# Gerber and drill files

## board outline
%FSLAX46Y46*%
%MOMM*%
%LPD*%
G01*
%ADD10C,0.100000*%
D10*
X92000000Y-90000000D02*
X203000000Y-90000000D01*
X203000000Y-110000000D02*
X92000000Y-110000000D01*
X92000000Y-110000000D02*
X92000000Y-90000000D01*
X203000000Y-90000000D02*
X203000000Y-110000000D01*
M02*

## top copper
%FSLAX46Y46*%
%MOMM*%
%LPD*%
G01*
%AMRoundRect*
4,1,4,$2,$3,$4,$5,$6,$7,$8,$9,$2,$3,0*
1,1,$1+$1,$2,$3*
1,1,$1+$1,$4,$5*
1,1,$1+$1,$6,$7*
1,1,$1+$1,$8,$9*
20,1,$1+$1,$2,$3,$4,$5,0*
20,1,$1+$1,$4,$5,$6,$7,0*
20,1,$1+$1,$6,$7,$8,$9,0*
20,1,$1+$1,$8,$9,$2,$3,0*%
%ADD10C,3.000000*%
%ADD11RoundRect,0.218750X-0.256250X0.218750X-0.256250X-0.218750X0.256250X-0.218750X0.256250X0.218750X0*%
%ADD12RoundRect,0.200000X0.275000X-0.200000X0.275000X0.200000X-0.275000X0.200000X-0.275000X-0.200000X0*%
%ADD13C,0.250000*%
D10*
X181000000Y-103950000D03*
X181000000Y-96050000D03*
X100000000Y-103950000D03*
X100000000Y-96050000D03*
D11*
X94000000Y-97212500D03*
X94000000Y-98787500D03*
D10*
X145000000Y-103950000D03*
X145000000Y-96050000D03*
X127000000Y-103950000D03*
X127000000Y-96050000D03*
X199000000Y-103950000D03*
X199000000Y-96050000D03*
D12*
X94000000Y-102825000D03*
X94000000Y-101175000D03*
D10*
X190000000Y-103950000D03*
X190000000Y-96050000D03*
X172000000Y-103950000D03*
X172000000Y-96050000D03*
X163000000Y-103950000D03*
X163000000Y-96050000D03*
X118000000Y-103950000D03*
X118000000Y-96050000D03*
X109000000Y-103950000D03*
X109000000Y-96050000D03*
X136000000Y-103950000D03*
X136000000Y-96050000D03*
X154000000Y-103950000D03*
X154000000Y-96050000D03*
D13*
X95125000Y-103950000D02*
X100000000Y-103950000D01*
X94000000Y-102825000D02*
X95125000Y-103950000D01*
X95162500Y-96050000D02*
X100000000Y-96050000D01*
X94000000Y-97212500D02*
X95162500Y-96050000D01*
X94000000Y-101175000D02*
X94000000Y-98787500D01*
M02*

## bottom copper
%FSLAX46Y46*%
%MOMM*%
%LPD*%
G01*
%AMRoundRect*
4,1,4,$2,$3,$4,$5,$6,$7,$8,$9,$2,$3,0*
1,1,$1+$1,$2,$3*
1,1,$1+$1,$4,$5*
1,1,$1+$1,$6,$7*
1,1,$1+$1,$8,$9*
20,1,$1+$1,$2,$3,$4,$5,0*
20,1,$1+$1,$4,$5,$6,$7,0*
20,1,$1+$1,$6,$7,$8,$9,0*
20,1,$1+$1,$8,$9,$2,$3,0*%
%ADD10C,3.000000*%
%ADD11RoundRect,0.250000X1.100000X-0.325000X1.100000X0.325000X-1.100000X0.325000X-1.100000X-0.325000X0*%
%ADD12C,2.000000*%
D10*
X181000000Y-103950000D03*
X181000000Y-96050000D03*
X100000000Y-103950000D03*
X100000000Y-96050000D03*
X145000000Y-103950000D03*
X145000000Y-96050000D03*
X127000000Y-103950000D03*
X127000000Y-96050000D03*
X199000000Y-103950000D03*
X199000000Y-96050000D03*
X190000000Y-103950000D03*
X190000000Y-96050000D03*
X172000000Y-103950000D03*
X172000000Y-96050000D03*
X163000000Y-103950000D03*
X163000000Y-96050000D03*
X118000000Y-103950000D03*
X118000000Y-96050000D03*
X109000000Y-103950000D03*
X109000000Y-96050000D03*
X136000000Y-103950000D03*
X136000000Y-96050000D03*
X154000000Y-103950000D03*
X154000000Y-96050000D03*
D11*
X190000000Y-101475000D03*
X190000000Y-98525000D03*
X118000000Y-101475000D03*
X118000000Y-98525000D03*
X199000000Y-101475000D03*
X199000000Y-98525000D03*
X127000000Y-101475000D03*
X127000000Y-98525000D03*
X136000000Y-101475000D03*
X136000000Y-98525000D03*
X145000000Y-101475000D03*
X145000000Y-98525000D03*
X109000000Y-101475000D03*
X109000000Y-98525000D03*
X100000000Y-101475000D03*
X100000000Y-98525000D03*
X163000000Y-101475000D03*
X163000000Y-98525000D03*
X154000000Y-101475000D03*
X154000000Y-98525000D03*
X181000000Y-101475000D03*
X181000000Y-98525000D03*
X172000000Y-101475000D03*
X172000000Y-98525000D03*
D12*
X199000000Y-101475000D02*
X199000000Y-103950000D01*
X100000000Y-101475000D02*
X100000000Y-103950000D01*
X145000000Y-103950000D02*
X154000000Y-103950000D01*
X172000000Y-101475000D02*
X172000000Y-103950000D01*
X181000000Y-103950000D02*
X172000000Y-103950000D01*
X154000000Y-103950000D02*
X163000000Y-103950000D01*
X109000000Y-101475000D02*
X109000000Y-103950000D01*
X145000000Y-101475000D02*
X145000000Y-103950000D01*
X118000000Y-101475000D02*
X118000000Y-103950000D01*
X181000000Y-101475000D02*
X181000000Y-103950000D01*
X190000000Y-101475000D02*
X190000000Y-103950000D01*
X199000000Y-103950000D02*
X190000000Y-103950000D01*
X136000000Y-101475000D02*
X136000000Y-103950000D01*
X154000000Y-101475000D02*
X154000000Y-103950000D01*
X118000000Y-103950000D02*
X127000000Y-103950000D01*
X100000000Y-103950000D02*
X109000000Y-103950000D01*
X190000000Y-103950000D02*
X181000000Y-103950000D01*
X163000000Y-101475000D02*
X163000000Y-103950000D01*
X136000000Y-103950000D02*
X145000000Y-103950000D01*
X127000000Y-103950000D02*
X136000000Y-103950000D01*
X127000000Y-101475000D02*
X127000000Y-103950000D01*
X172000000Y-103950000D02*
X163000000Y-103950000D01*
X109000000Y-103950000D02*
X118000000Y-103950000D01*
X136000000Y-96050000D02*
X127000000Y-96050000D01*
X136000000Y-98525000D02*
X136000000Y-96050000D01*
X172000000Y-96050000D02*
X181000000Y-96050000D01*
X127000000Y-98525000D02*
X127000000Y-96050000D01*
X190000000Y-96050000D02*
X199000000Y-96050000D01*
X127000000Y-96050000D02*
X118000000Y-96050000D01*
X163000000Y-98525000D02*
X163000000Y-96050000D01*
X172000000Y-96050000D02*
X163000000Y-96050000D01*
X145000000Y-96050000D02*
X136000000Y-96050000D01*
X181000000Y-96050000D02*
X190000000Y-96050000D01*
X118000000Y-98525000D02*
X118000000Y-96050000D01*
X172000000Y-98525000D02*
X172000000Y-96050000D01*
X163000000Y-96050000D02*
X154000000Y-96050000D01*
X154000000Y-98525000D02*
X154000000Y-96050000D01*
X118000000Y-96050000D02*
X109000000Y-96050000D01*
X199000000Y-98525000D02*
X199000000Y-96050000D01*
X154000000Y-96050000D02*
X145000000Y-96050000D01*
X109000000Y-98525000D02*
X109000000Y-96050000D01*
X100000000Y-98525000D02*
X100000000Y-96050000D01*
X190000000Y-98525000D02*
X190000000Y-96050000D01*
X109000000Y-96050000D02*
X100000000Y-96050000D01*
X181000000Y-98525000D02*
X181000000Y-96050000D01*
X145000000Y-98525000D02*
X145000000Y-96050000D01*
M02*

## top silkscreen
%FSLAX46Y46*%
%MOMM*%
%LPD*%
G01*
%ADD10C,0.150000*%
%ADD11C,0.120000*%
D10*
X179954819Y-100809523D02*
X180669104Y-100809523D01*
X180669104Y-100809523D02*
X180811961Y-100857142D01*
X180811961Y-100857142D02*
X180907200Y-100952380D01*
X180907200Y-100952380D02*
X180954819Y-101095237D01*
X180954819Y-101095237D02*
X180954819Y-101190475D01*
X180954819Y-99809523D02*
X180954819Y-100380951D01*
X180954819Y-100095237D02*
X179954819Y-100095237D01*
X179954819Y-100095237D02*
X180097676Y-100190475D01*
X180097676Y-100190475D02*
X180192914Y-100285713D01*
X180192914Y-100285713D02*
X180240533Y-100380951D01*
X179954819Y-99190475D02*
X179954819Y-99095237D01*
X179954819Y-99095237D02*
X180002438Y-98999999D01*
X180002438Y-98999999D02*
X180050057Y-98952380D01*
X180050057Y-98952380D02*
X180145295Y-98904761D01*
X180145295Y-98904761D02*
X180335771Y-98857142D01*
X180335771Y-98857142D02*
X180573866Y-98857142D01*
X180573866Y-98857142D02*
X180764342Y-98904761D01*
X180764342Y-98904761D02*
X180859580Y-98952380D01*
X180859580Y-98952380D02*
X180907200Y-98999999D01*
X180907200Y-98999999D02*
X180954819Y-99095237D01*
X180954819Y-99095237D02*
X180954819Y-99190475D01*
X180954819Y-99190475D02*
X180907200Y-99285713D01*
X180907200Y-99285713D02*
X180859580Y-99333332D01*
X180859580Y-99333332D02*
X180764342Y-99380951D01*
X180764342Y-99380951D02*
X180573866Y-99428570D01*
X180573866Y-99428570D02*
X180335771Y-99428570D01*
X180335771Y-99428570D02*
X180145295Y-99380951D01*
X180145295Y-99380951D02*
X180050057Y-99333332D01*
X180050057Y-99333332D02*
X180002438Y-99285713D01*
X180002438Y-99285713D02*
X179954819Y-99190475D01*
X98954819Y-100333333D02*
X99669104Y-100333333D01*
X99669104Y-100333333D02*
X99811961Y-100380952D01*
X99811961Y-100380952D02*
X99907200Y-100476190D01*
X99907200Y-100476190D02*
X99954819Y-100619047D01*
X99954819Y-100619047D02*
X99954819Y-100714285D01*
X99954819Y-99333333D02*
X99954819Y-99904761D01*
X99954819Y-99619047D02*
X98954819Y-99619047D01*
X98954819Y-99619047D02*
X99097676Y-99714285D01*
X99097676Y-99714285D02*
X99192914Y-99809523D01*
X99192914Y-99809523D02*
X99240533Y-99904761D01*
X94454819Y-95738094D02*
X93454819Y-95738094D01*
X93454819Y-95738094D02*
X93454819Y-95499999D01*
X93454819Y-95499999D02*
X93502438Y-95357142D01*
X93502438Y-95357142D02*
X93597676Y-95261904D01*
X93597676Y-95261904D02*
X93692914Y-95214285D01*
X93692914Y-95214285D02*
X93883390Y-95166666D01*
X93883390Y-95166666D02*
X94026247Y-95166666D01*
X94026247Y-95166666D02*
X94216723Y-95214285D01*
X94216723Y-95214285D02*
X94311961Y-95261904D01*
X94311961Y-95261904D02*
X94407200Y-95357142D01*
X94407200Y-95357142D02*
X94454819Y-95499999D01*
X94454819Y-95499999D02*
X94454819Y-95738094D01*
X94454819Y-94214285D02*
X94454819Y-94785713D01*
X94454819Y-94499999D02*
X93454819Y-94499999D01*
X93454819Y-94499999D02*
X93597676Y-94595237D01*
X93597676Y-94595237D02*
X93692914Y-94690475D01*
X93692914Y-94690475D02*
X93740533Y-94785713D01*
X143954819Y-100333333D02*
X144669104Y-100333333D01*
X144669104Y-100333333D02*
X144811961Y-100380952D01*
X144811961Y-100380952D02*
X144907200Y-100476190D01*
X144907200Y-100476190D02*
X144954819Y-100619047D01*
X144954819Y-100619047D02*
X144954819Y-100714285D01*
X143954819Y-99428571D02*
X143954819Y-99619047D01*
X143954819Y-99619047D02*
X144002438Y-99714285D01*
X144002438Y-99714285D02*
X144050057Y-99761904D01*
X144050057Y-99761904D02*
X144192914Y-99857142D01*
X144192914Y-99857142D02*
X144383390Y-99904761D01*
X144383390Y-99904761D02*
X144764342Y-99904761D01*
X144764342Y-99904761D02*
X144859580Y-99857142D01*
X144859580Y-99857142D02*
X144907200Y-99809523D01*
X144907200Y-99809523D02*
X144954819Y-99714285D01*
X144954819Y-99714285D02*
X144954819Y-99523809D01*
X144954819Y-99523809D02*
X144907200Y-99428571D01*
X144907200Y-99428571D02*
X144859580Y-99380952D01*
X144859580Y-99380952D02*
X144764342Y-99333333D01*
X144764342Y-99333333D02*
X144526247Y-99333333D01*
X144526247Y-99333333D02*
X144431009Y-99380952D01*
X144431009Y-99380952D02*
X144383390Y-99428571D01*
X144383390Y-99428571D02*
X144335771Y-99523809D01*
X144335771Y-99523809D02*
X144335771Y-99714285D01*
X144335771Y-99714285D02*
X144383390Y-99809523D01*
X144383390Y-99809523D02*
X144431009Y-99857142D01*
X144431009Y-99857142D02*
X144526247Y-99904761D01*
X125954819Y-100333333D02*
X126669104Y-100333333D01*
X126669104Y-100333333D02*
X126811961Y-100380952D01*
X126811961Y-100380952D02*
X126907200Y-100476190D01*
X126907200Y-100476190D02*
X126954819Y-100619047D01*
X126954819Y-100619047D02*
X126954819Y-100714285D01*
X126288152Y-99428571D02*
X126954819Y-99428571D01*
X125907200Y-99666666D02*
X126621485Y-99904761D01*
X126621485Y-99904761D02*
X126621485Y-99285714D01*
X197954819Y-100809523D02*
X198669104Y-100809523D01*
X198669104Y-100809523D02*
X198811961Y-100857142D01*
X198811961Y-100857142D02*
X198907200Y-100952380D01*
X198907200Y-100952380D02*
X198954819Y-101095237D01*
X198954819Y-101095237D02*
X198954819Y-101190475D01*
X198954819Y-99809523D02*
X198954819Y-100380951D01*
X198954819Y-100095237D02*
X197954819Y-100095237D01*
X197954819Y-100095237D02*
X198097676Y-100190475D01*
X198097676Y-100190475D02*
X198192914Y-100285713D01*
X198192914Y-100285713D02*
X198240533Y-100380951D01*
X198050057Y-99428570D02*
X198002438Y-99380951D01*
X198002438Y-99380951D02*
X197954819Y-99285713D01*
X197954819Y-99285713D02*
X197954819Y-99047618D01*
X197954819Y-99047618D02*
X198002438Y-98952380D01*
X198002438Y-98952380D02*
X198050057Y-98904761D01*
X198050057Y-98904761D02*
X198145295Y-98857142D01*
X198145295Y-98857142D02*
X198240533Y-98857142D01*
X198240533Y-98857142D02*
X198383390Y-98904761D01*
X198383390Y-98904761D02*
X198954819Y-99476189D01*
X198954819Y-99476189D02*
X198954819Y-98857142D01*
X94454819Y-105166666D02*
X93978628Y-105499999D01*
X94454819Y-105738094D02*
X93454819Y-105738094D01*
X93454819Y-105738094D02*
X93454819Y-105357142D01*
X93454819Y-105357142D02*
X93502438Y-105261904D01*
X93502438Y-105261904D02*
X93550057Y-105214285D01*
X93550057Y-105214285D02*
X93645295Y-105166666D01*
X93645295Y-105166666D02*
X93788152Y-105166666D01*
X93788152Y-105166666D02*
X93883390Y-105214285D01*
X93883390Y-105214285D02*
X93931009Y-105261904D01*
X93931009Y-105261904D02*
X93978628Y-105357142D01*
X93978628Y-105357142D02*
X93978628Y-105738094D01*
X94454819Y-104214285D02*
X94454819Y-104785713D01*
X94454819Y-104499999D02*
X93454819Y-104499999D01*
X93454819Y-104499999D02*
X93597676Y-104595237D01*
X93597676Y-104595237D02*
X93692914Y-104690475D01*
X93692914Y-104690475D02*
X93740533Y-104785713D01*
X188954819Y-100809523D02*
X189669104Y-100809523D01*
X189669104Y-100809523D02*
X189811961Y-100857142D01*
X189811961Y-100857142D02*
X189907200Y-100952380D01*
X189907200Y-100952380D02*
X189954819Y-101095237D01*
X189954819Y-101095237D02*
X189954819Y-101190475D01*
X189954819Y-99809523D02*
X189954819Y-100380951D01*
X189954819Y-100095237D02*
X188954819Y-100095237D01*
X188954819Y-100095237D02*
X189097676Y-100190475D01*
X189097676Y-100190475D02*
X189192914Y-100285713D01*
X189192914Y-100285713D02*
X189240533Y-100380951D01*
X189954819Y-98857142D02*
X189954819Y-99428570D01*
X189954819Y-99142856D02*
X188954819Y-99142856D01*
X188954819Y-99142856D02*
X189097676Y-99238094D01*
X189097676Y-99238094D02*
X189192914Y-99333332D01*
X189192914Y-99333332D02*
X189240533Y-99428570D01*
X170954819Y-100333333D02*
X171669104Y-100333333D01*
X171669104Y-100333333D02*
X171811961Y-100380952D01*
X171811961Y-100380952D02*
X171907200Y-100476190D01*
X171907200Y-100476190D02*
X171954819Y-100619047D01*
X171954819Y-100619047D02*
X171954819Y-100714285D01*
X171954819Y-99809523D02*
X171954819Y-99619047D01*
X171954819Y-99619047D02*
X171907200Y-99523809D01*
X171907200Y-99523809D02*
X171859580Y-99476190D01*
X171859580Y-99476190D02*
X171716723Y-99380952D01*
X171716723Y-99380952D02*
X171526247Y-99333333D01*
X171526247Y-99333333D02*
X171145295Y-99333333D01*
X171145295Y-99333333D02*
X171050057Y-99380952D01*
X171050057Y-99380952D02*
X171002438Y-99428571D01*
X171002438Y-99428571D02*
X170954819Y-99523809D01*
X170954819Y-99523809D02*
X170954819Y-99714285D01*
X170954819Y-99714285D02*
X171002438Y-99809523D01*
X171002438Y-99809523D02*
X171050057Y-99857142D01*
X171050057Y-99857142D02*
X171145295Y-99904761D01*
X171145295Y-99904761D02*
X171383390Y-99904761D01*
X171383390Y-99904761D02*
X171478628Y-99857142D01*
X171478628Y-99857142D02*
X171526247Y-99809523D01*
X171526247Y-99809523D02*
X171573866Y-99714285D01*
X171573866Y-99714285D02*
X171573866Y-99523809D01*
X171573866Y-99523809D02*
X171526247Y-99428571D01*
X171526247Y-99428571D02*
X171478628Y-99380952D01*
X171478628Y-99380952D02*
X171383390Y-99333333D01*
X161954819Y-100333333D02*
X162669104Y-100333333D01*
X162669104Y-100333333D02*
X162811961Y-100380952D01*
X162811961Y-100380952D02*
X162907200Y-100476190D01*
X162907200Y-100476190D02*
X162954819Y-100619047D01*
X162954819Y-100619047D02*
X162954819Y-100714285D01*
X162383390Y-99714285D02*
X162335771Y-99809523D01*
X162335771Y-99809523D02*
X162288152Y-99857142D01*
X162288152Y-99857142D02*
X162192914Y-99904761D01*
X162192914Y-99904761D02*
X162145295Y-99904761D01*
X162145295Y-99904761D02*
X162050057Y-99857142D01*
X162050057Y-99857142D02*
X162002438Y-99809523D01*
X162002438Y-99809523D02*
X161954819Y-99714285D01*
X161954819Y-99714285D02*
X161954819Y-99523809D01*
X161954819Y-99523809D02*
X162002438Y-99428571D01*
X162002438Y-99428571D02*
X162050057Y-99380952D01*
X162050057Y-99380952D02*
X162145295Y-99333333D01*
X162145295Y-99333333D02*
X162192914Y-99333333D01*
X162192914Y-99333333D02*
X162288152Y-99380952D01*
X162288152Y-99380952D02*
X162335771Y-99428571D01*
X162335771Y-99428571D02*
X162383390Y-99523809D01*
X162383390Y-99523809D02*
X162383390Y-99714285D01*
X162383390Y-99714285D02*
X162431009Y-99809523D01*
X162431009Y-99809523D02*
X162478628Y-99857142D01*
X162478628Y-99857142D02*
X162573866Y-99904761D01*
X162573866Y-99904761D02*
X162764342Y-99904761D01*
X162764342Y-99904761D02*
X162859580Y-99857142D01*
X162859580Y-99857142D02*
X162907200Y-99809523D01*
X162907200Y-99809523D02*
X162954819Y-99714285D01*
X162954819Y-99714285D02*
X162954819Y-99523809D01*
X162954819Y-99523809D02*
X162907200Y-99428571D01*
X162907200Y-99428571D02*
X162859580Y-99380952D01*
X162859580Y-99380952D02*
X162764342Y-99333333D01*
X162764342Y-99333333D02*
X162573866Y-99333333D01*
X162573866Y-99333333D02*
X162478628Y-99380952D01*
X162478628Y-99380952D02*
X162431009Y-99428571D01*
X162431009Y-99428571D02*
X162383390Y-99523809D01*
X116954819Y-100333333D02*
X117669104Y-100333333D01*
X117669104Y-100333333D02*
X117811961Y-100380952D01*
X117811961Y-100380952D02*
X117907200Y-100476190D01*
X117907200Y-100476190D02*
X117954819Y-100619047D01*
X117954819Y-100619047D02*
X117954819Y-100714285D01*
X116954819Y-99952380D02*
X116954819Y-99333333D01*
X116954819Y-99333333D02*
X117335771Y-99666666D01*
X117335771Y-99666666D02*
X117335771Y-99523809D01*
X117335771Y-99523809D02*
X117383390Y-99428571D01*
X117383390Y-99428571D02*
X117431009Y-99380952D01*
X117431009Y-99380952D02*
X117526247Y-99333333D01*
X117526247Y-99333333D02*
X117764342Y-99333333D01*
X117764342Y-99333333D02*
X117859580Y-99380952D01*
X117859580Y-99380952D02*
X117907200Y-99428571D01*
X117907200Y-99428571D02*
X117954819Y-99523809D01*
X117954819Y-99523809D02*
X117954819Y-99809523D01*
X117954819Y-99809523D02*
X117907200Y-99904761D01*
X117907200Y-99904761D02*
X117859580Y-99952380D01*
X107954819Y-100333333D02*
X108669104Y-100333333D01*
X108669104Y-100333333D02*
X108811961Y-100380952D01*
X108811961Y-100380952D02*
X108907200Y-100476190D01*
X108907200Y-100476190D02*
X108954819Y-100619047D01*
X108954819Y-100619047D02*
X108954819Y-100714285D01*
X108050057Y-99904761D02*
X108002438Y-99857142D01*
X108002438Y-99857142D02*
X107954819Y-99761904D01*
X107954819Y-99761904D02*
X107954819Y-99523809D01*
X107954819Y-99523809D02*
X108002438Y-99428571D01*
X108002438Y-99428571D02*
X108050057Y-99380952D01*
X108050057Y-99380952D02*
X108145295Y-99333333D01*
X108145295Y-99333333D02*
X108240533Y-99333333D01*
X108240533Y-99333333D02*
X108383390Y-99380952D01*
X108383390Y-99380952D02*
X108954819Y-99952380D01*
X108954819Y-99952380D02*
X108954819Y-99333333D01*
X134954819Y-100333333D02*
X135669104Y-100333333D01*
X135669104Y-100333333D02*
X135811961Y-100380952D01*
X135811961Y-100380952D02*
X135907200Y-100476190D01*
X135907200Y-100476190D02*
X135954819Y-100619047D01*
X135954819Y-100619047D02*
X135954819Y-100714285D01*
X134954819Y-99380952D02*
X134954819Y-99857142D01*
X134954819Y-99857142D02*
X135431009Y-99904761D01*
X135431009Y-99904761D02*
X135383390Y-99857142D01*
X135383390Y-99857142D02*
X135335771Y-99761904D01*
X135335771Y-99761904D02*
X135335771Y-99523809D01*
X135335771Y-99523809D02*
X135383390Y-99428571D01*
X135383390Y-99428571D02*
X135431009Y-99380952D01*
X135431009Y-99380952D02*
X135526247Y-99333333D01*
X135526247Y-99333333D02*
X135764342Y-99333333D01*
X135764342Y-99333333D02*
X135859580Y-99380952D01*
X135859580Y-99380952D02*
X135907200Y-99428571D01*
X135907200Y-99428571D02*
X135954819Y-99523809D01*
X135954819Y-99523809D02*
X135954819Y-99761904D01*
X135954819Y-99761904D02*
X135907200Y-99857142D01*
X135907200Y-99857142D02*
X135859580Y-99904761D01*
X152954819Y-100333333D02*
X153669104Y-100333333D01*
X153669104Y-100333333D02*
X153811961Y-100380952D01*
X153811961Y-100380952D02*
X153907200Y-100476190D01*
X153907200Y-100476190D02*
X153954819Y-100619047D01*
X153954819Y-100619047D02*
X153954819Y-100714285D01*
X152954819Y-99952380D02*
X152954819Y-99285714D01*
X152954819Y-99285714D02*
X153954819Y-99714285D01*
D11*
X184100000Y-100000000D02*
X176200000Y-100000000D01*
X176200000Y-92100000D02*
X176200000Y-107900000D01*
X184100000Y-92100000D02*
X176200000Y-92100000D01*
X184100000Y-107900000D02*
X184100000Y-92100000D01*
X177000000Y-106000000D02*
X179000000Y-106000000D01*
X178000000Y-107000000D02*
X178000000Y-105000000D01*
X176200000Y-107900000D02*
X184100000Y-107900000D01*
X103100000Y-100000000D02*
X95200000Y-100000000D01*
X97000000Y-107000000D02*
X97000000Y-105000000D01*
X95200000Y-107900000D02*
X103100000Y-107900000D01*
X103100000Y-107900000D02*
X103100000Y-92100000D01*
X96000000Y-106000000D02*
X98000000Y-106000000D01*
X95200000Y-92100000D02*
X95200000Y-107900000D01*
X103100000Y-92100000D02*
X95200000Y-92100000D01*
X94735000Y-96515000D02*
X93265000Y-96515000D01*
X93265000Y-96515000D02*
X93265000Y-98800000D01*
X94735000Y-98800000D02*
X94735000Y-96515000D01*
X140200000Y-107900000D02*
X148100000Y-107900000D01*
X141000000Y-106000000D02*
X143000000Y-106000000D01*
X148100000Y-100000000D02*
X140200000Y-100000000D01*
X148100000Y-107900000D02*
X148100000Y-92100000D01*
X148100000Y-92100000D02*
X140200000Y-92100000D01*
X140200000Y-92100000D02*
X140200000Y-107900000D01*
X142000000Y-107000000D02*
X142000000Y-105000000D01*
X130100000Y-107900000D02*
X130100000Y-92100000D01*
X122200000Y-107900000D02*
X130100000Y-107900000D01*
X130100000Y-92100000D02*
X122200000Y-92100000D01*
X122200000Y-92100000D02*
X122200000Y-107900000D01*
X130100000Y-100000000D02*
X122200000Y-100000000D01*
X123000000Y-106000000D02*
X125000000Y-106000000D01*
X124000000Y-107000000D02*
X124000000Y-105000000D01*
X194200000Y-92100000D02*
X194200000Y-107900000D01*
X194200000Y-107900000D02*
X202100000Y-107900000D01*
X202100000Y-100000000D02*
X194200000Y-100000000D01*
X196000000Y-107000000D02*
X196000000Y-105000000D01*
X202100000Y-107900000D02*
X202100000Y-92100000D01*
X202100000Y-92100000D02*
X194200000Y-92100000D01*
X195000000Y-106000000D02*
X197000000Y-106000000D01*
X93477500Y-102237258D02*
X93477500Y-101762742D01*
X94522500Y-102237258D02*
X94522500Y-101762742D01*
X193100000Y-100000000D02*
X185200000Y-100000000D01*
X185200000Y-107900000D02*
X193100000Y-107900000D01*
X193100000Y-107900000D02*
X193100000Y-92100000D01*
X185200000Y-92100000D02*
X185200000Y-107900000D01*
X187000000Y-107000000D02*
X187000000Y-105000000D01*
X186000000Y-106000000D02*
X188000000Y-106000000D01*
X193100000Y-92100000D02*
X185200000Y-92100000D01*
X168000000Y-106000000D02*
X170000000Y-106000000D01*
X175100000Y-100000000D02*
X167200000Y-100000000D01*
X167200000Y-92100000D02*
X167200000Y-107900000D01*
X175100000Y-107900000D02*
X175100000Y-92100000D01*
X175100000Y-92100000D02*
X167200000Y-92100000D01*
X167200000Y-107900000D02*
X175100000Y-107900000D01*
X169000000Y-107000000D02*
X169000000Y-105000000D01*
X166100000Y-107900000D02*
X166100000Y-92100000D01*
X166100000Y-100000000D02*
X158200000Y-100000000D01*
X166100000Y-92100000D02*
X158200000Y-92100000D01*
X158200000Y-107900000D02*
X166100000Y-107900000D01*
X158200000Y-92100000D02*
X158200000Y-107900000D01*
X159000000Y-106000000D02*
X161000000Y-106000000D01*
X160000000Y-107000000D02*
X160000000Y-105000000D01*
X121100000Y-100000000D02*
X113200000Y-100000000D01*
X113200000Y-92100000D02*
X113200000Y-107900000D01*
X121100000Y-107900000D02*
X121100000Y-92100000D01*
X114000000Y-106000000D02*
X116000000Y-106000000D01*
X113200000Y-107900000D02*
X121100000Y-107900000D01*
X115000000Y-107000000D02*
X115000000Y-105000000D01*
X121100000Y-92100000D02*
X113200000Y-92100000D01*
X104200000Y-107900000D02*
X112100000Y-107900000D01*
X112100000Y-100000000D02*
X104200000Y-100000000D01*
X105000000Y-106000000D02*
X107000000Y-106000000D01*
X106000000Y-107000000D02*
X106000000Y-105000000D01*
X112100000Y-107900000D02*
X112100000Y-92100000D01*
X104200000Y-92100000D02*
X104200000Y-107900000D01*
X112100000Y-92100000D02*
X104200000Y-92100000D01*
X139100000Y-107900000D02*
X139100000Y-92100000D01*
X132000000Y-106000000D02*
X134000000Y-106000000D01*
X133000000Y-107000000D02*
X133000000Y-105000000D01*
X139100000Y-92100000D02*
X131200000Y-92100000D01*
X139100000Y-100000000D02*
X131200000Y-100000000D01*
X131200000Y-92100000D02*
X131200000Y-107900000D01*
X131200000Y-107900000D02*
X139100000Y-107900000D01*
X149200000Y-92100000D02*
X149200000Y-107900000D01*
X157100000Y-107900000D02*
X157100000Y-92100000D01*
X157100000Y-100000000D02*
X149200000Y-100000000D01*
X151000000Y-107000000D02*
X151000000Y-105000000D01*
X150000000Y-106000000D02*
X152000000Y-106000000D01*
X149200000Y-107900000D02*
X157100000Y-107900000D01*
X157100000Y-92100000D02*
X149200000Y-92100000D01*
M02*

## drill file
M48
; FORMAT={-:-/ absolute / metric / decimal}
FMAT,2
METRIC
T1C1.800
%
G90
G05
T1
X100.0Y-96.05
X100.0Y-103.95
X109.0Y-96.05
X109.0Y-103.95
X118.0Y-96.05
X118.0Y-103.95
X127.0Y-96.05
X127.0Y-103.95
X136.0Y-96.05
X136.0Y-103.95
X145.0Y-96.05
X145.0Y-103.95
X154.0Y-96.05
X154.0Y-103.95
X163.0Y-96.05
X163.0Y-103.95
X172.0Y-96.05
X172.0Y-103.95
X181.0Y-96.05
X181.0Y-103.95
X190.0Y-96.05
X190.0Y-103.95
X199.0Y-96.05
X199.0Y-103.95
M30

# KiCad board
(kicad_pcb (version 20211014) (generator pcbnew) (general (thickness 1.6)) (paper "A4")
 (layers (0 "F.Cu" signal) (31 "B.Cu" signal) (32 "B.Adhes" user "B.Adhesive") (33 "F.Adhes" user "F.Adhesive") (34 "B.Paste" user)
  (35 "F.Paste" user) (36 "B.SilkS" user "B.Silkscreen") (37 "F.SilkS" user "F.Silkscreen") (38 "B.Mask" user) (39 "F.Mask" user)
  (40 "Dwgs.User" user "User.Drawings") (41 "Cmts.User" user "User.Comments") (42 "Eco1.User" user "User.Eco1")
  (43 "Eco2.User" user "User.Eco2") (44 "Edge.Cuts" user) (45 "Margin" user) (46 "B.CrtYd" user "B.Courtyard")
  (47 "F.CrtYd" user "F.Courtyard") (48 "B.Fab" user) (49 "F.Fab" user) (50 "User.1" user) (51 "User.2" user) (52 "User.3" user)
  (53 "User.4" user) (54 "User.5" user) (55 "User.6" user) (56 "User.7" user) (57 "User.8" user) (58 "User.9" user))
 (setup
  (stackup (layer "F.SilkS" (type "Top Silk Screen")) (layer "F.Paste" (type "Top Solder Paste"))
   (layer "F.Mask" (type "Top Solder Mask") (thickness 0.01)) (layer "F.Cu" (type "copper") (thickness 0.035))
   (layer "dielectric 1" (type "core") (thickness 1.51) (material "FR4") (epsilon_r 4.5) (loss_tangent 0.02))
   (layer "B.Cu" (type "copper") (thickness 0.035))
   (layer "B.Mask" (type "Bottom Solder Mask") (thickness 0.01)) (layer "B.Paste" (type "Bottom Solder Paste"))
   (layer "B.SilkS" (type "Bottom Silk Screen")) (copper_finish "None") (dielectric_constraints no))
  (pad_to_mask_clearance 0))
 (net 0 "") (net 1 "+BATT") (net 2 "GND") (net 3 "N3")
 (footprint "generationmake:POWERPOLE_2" (layer "F.Cu") (at 181 100 90)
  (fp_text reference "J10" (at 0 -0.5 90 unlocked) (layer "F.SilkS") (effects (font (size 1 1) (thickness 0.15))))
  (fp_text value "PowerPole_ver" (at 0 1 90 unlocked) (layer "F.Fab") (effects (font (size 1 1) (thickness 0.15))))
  (fp_line (start 0 3.1) (end 0 -4.8) (layer "F.SilkS") (width 0.12))
  (fp_line (start 7.9 -4.8) (end -7.9 -4.8) (layer "F.SilkS") (width 0.12))
  (fp_line (start 7.9 3.1) (end 7.9 -4.8) (layer "F.SilkS") (width 0.12))
  (fp_line (start -7.9 3.1) (end 7.9 3.1) (layer "F.SilkS") (width 0.12))
  (fp_line (start -6 -4) (end -6 -2) (layer "F.SilkS") (width 0.12))
  (fp_line (start -7 -3) (end -5 -3) (layer "F.SilkS") (width 0.12))
  (fp_line (start -7.9 -4.8) (end -7.9 3.1) (layer "F.SilkS") (width 0.12))
  (pad "1" thru_hole circle (at -3.95 0 90) (size 3 3) (drill 1.8) (layers *.Cu *.Mask) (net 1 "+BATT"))
  (pad "2" thru_hole circle (at 3.95 0 90) (size 3 3) (drill 1.8) (layers *.Cu *.Mask) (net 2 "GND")))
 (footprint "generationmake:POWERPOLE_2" (layer "F.Cu") (at 100 100 90)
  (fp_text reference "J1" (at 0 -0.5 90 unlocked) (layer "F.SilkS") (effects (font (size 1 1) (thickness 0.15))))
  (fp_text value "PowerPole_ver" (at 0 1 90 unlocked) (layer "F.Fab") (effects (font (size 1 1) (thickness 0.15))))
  (fp_line (start 0 3.1) (end 0 -4.8) (layer "F.SilkS") (width 0.12))
  (fp_line (start -7 -3) (end -5 -3) (layer "F.SilkS") (width 0.12))
  (fp_line (start -7.9 -4.8) (end -7.9 3.1) (layer "F.SilkS") (width 0.12))
  (fp_line (start -7.9 3.1) (end 7.9 3.1) (layer "F.SilkS") (width 0.12))
  (fp_line (start -6 -4) (end -6 -2) (layer "F.SilkS") (width 0.12))
  (fp_line (start 7.9 -4.8) (end -7.9 -4.8) (layer "F.SilkS") (width 0.12))
  (fp_line (start 7.9 3.1) (end 7.9 -4.8) (layer "F.SilkS") (width 0.12))
  (pad "1" thru_hole circle (at -3.95 0 90) (size 3 3) (drill 1.8) (layers *.Cu *.Mask) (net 1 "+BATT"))
  (pad "2" thru_hole circle (at 3.95 0 90) (size 3 3) (drill 1.8) (layers *.Cu *.Mask) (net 2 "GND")))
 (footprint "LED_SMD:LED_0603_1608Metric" (layer "F.Cu") (at 94 98 -90)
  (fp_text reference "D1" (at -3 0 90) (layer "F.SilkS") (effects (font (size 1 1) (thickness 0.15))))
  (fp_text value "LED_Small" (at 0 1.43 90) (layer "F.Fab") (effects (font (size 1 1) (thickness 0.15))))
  (fp_line (start -1.485 -0.735) (end -1.485 0.735) (layer "F.SilkS") (width 0.12))
  (fp_line (start -1.485 0.735) (end 0.8 0.735) (layer "F.SilkS") (width 0.12))
  (fp_line (start 0.8 -0.735) (end -1.485 -0.735) (layer "F.SilkS") (width 0.12))
  (pad "1" smd roundrect (at -0.7875 0 270) (size 0.875 0.95) (layers "F.Cu" "F.Paste" "F.Mask") (roundrect_rratio 0.25) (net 2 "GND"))
  (pad "2" smd roundrect (at 0.7875 0 270) (size 0.875 0.95) (layers "F.Cu" "F.Paste" "F.Mask") (roundrect_rratio 0.25) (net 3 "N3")))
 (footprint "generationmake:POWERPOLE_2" (layer "F.Cu") (at 145 100 90)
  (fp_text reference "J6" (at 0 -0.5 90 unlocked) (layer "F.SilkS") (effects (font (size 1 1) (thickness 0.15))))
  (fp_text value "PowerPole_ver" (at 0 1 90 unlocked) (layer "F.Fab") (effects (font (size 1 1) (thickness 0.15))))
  (fp_line (start -7.9 -4.8) (end -7.9 3.1) (layer "F.SilkS") (width 0.12))
  (fp_line (start -6 -4) (end -6 -2) (layer "F.SilkS") (width 0.12))
  (fp_line (start 0 3.1) (end 0 -4.8) (layer "F.SilkS") (width 0.12))
  (fp_line (start -7.9 3.1) (end 7.9 3.1) (layer "F.SilkS") (width 0.12))
  (fp_line (start 7.9 3.1) (end 7.9 -4.8) (layer "F.SilkS") (width 0.12))
  (fp_line (start 7.9 -4.8) (end -7.9 -4.8) (layer "F.SilkS") (width 0.12))
  (fp_line (start -7 -3) (end -5 -3) (layer "F.SilkS") (width 0.12))
  (pad "1" thru_hole circle (at -3.95 0 90) (size 3 3) (drill 1.8) (layers *.Cu *.Mask) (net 1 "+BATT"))
  (pad "2" thru_hole circle (at 3.95 0 90) (size 3 3) (drill 1.8) (layers *.Cu *.Mask) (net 2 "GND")))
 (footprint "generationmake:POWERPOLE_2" (layer "F.Cu") (at 127 100 90)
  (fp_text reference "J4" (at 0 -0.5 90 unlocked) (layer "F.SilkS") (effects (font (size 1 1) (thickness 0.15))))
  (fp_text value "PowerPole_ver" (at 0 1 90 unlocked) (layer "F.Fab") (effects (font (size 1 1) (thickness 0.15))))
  (fp_line (start -7.9 3.1) (end 7.9 3.1) (layer "F.SilkS") (width 0.12))
  (fp_line (start -7.9 -4.8) (end -7.9 3.1) (layer "F.SilkS") (width 0.12))
  (fp_line (start 7.9 3.1) (end 7.9 -4.8) (layer "F.SilkS") (width 0.12))
  (fp_line (start 7.9 -4.8) (end -7.9 -4.8) (layer "F.SilkS") (width 0.12))
  (fp_line (start 0 3.1) (end 0 -4.8) (layer "F.SilkS") (width 0.12))
  (fp_line (start -6 -4) (end -6 -2) (layer "F.SilkS") (width 0.12))
  (fp_line (start -7 -3) (end -5 -3) (layer "F.SilkS") (width 0.12))
  (pad "1" thru_hole circle (at -3.95 0 90) (size 3 3) (drill 1.8) (layers *.Cu *.Mask) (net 1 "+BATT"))
  (pad "2" thru_hole circle (at 3.95 0 90) (size 3 3) (drill 1.8) (layers *.Cu *.Mask) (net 2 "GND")))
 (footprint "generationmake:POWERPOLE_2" (layer "F.Cu") (at 199 100 90)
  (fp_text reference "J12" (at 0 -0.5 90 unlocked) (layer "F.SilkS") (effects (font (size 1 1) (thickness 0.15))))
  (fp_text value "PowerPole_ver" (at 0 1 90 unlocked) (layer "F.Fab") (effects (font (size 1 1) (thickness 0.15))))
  (fp_line (start 7.9 -4.8) (end -7.9 -4.8) (layer "F.SilkS") (width 0.12))
  (fp_line (start -7.9 -4.8) (end -7.9 3.1) (layer "F.SilkS") (width 0.12))
  (fp_line (start 0 3.1) (end 0 -4.8) (layer "F.SilkS") (width 0.12))
  (fp_line (start -7 -3) (end -5 -3) (layer "F.SilkS") (width 0.12))
  (fp_line (start -7.9 3.1) (end 7.9 3.1) (layer "F.SilkS") (width 0.12))
  (fp_line (start 7.9 3.1) (end 7.9 -4.8) (layer "F.SilkS") (width 0.12))
  (fp_line (start -6 -4) (end -6 -2) (layer "F.SilkS") (width 0.12))
  (pad "1" thru_hole circle (at -3.95 0 90) (size 3 3) (drill 1.8) (layers *.Cu *.Mask) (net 1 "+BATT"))
  (pad "2" thru_hole circle (at 3.95 0 90) (size 3 3) (drill 1.8) (layers *.Cu *.Mask) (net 2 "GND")))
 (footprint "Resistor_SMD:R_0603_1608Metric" (layer "F.Cu") (at 94 102 90)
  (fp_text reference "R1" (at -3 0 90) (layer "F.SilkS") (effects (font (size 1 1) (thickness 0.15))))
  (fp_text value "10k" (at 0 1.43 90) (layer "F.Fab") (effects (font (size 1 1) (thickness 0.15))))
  (fp_line (start -0.237258 -0.5225) (end 0.237258 -0.5225) (layer "F.SilkS") (width 0.12))
  (fp_line (start -0.237258 0.5225) (end 0.237258 0.5225) (layer "F.SilkS") (width 0.12))
  (pad "1" smd roundrect (at -0.825 0 90) (size 0.8 0.95) (layers "F.Cu" "F.Paste" "F.Mask") (roundrect_rratio 0.25) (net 1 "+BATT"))
  (pad "2" smd roundrect (at 0.825 0 90) (size 0.8 0.95) (layers "F.Cu" "F.Paste" "F.Mask") (roundrect_rratio 0.25) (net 3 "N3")))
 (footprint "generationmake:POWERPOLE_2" (layer "F.Cu") (at 190 100 90)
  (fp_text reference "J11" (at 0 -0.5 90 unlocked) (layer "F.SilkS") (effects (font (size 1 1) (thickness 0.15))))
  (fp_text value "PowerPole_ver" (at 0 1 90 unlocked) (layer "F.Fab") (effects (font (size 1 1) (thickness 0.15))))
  (fp_line (start 0 3.1) (end 0 -4.8) (layer "F.SilkS") (width 0.12))
  (fp_line (start -7.9 -4.8) (end -7.9 3.1) (layer "F.SilkS") (width 0.12))
  (fp_line (start -7.9 3.1) (end 7.9 3.1) (layer "F.SilkS") (width 0.12))
  (fp_line (start 7.9 -4.8) (end -7.9 -4.8) (layer "F.SilkS") (width 0.12))
  (fp_line (start -7 -3) (end -5 -3) (layer "F.SilkS") (width 0.12))
  (fp_line (start -6 -4) (end -6 -2) (layer "F.SilkS") (width 0.12))
  (fp_line (start 7.9 3.1) (end 7.9 -4.8) (layer "F.SilkS") (width 0.12))
  (pad "1" thru_hole circle (at -3.95 0 90) (size 3 3) (drill 1.8) (layers *.Cu *.Mask) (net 1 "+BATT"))
  (pad "2" thru_hole circle (at 3.95 0 90) (size 3 3) (drill 1.8) (layers *.Cu *.Mask) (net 2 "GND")))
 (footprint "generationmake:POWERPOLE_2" (layer "F.Cu") (at 172 100 90)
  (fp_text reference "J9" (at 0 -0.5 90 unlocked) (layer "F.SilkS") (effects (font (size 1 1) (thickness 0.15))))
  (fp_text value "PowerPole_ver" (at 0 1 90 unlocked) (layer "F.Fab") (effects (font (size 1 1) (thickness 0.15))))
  (fp_line (start -6 -4) (end -6 -2) (layer "F.SilkS") (width 0.12))
  (fp_line (start 0 3.1) (end 0 -4.8) (layer "F.SilkS") (width 0.12))
  (fp_line (start 7.9 -4.8) (end -7.9 -4.8) (layer "F.SilkS") (width 0.12))
  (fp_line (start -7.9 3.1) (end 7.9 3.1) (layer "F.SilkS") (width 0.12))
  (fp_line (start 7.9 3.1) (end 7.9 -4.8) (layer "F.SilkS") (width 0.12))
  (fp_line (start -7.9 -4.8) (end -7.9 3.1) (layer "F.SilkS") (width 0.12))
  (fp_line (start -7 -3) (end -5 -3) (layer "F.SilkS") (width 0.12))
  (pad "1" thru_hole circle (at -3.95 0 90) (size 3 3) (drill 1.8) (layers *.Cu *.Mask) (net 1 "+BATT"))
  (pad "2" thru_hole circle (at 3.95 0 90) (size 3 3) (drill 1.8) (layers *.Cu *.Mask) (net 2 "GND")))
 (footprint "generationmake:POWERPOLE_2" (layer "F.Cu") (at 163 100 90)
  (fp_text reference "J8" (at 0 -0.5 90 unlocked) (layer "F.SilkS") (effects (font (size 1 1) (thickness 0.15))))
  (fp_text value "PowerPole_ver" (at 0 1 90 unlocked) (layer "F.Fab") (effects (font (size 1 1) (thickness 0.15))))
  (fp_line (start -7.9 3.1) (end 7.9 3.1) (layer "F.SilkS") (width 0.12))
  (fp_line (start 0 3.1) (end 0 -4.8) (layer "F.SilkS") (width 0.12))
  (fp_line (start 7.9 3.1) (end 7.9 -4.8) (layer "F.SilkS") (width 0.12))
  (fp_line (start -7.9 -4.8) (end -7.9 3.1) (layer "F.SilkS") (width 0.12))
  (fp_line (start 7.9 -4.8) (end -7.9 -4.8) (layer "F.SilkS") (width 0.12))
  (fp_line (start -6 -4) (end -6 -2) (layer "F.SilkS") (width 0.12))
  (fp_line (start -7 -3) (end -5 -3) (layer "F.SilkS") (width 0.12))
  (pad "1" thru_hole circle (at -3.95 0 90) (size 3 3) (drill 1.8) (layers *.Cu *.Mask) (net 1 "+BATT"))
  (pad "2" thru_hole circle (at 3.95 0 90) (size 3 3) (drill 1.8) (layers *.Cu *.Mask) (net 2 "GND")))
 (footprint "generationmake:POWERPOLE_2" (layer "F.Cu") (at 118 100 90)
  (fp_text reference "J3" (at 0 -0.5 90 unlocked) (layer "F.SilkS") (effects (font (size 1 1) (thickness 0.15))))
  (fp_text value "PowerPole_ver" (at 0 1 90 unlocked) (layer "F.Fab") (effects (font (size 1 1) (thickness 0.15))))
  (fp_line (start 0 3.1) (end 0 -4.8) (layer "F.SilkS") (width 0.12))
  (fp_line (start 7.9 -4.8) (end -7.9 -4.8) (layer "F.SilkS") (width 0.12))
  (fp_line (start -7.9 3.1) (end 7.9 3.1) (layer "F.SilkS") (width 0.12))
  (fp_line (start -6 -4) (end -6 -2) (layer "F.SilkS") (width 0.12))
  (fp_line (start -7.9 -4.8) (end -7.9 3.1) (layer "F.SilkS") (width 0.12))
  (fp_line (start -7 -3) (end -5 -3) (layer "F.SilkS") (width 0.12))
  (fp_line (start 7.9 3.1) (end 7.9 -4.8) (layer "F.SilkS") (width 0.12))
  (pad "1" thru_hole circle (at -3.95 0 90) (size 3 3) (drill 1.8) (layers *.Cu *.Mask) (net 1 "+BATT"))
  (pad "2" thru_hole circle (at 3.95 0 90) (size 3 3) (drill 1.8) (layers *.Cu *.Mask) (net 2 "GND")))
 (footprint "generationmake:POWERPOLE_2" (layer "F.Cu") (at 109 100 90)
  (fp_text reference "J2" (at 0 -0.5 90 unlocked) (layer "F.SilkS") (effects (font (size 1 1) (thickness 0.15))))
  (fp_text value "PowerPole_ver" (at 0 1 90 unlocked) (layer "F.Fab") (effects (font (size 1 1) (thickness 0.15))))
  (fp_line (start -7.9 -4.8) (end -7.9 3.1) (layer "F.SilkS") (width 0.12))
  (fp_line (start 0 3.1) (end 0 -4.8) (layer "F.SilkS") (width 0.12))
  (fp_line (start -6 -4) (end -6 -2) (layer "F.SilkS") (width 0.12))
  (fp_line (start -7 -3) (end -5 -3) (layer "F.SilkS") (width 0.12))
  (fp_line (start -7.9 3.1) (end 7.9 3.1) (layer "F.SilkS") (width 0.12))
  (fp_line (start 7.9 -4.8) (end -7.9 -4.8) (layer "F.SilkS") (width 0.12))
  (fp_line (start 7.9 3.1) (end 7.9 -4.8) (layer "F.SilkS") (width 0.12))
  (pad "1" thru_hole circle (at -3.95 0 90) (size 3 3) (drill 1.8) (layers *.Cu *.Mask) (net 1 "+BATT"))
  (pad "2" thru_hole circle (at 3.95 0 90) (size 3 3) (drill 1.8) (layers *.Cu *.Mask) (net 2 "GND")))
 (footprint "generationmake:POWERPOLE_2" (layer "F.Cu") (at 136 100 90)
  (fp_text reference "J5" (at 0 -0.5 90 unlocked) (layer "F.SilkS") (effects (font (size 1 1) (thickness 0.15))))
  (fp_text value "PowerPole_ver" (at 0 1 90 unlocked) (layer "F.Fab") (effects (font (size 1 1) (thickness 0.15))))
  (fp_line (start -7.9 3.1) (end 7.9 3.1) (layer "F.SilkS") (width 0.12))
  (fp_line (start -6 -4) (end -6 -2) (layer "F.SilkS") (width 0.12))
  (fp_line (start -7 -3) (end -5 -3) (layer "F.SilkS") (width 0.12))
  (fp_line (start 7.9 3.1) (end 7.9 -4.8) (layer "F.SilkS") (width 0.12))
  (fp_line (start 0 3.1) (end 0 -4.8) (layer "F.SilkS") (width 0.12))
  (fp_line (start 7.9 -4.8) (end -7.9 -4.8) (layer "F.SilkS") (width 0.12))
  (fp_line (start -7.9 -4.8) (end -7.9 3.1) (layer "F.SilkS") (width 0.12))
  (pad "1" thru_hole circle (at -3.95 0 90) (size 3 3) (drill 1.8) (layers *.Cu *.Mask) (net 1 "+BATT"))
  (pad "2" thru_hole circle (at 3.95 0 90) (size 3 3) (drill 1.8) (layers *.Cu *.Mask) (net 2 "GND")))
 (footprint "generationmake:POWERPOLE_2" (layer "F.Cu") (at 154 100 90)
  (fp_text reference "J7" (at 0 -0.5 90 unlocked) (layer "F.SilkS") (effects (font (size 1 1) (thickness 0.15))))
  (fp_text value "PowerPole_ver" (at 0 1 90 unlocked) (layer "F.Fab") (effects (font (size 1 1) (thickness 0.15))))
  (fp_line (start 7.9 -4.8) (end -7.9 -4.8) (layer "F.SilkS") (width 0.12))
  (fp_line (start -7.9 3.1) (end 7.9 3.1) (layer "F.SilkS") (width 0.12))
  (fp_line (start 0 3.1) (end 0 -4.8) (layer "F.SilkS") (width 0.12))
  (fp_line (start -7 -3) (end -5 -3) (layer "F.SilkS") (width 0.12))
  (fp_line (start -6 -4) (end -6 -2) (layer "F.SilkS") (width 0.12))
  (fp_line (start -7.9 -4.8) (end -7.9 3.1) (layer "F.SilkS") (width 0.12))
  (fp_line (start 7.9 3.1) (end 7.9 -4.8) (layer "F.SilkS") (width 0.12))
  (pad "1" thru_hole circle (at -3.95 0 90) (size 3 3) (drill 1.8) (layers *.Cu *.Mask) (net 1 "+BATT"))
  (pad "2" thru_hole circle (at 3.95 0 90) (size 3 3) (drill 1.8) (layers *.Cu *.Mask) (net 2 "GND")))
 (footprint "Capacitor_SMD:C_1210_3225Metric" (layer "B.Cu") (at 190 100 90)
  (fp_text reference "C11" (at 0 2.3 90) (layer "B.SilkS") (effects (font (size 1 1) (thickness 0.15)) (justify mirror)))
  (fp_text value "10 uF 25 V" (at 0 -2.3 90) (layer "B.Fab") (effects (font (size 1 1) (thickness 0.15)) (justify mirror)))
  (pad "1" smd roundrect (at -1.475 0 90) (size 1.15 2.7) (layers "B.Cu" "B.Paste" "B.Mask") (roundrect_rratio 0.217391) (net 1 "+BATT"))
  (pad "2" smd roundrect (at 1.475 0 90) (size 1.15 2.7) (layers "B.Cu" "B.Paste" "B.Mask") (roundrect_rratio 0.217391) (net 2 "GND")))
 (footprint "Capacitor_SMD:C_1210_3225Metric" (layer "B.Cu") (at 118 100 90)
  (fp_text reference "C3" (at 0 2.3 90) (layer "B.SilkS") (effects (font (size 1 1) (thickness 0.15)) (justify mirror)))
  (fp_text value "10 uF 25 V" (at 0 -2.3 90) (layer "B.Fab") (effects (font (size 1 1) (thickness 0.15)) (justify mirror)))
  (pad "1" smd roundrect (at -1.475 0 90) (size 1.15 2.7) (layers "B.Cu" "B.Paste" "B.Mask") (roundrect_rratio 0.217391) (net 1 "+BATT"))
  (pad "2" smd roundrect (at 1.475 0 90) (size 1.15 2.7) (layers "B.Cu" "B.Paste" "B.Mask") (roundrect_rratio 0.217391) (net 2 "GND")))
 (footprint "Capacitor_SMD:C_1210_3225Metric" (layer "B.Cu") (at 199 100 90)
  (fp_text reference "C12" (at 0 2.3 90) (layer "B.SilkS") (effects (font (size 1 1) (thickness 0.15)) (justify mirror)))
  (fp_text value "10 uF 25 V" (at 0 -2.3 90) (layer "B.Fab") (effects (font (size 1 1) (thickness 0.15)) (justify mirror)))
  (pad "1" smd roundrect (at -1.475 0 90) (size 1.15 2.7) (layers "B.Cu" "B.Paste" "B.Mask") (roundrect_rratio 0.217391) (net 1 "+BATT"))
  (pad "2" smd roundrect (at 1.475 0 90) (size 1.15 2.7) (layers "B.Cu" "B.Paste" "B.Mask") (roundrect_rratio 0.217391) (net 2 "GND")))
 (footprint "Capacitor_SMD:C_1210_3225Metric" (layer "B.Cu") (at 127 100 90)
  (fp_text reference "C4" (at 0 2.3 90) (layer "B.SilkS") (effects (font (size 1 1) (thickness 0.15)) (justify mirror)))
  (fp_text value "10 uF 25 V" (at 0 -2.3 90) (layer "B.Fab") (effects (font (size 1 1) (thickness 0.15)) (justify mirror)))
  (pad "1" smd roundrect (at -1.475 0 90) (size 1.15 2.7) (layers "B.Cu" "B.Paste" "B.Mask") (roundrect_rratio 0.217391) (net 1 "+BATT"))
  (pad "2" smd roundrect (at 1.475 0 90) (size 1.15 2.7) (layers "B.Cu" "B.Paste" "B.Mask") (roundrect_rratio 0.217391) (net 2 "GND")))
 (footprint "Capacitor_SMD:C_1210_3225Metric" (layer "B.Cu") (at 136 100 90)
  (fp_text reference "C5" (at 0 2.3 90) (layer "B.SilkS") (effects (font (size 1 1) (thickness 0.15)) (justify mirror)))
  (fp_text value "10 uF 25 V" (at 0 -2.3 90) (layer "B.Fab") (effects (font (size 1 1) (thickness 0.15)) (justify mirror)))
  (pad "1" smd roundrect (at -1.475 0 90) (size 1.15 2.7) (layers "B.Cu" "B.Paste" "B.Mask") (roundrect_rratio 0.217391) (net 1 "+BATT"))
  (pad "2" smd roundrect (at 1.475 0 90) (size 1.15 2.7) (layers "B.Cu" "B.Paste" "B.Mask") (roundrect_rratio 0.217391) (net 2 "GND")))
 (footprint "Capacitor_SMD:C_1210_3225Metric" (layer "B.Cu") (at 145 100 90)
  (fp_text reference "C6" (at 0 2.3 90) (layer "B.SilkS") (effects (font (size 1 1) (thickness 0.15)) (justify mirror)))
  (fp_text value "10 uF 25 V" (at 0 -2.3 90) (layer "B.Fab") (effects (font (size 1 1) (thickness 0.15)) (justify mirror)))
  (pad "1" smd roundrect (at -1.475 0 90) (size 1.15 2.7) (layers "B.Cu" "B.Paste" "B.Mask") (roundrect_rratio 0.217391) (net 1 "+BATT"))
  (pad "2" smd roundrect (at 1.475 0 90) (size 1.15 2.7) (layers "B.Cu" "B.Paste" "B.Mask") (roundrect_rratio 0.217391) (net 2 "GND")))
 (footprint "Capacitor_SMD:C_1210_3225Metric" (layer "B.Cu") (at 109 100 90)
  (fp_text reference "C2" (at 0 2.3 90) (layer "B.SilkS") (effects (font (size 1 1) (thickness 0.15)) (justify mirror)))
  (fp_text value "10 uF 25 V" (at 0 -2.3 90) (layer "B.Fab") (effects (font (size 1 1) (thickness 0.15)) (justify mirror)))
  (pad "1" smd roundrect (at -1.475 0 90) (size 1.15 2.7) (layers "B.Cu" "B.Paste" "B.Mask") (roundrect_rratio 0.217391) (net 1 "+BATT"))
  (pad "2" smd roundrect (at 1.475 0 90) (size 1.15 2.7) (layers "B.Cu" "B.Paste" "B.Mask") (roundrect_rratio 0.217391) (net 2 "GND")))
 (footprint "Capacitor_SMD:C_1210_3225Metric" (layer "B.Cu") (at 100 100 90)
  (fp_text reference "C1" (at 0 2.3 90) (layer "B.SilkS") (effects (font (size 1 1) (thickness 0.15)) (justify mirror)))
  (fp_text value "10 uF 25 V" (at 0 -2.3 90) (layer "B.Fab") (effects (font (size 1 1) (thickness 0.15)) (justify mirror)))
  (pad "1" smd roundrect (at -1.475 0 90) (size 1.15 2.7) (layers "B.Cu" "B.Paste" "B.Mask") (roundrect_rratio 0.217391) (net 1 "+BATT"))
  (pad "2" smd roundrect (at 1.475 0 90) (size 1.15 2.7) (layers "B.Cu" "B.Paste" "B.Mask") (roundrect_rratio 0.217391) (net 2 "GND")))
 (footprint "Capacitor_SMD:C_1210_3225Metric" (layer "B.Cu") (at 163 100 90)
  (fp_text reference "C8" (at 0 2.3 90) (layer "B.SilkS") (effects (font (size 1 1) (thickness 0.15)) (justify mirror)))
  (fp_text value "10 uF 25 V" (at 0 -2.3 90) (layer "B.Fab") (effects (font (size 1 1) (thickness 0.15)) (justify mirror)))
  (pad "1" smd roundrect (at -1.475 0 90) (size 1.15 2.7) (layers "B.Cu" "B.Paste" "B.Mask") (roundrect_rratio 0.217391) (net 1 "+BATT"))
  (pad "2" smd roundrect (at 1.475 0 90) (size 1.15 2.7) (layers "B.Cu" "B.Paste" "B.Mask") (roundrect_rratio 0.217391) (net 2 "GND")))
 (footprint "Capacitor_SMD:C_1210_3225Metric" (layer "B.Cu") (at 154 100 90)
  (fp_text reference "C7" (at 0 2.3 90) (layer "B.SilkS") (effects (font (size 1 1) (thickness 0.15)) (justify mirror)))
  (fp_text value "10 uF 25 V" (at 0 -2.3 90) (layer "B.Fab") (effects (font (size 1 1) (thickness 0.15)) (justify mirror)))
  (pad "1" smd roundrect (at -1.475 0 90) (size 1.15 2.7) (layers "B.Cu" "B.Paste" "B.Mask") (roundrect_rratio 0.217391) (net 1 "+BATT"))
  (pad "2" smd roundrect (at 1.475 0 90) (size 1.15 2.7) (layers "B.Cu" "B.Paste" "B.Mask") (roundrect_rratio 0.217391) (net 2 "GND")))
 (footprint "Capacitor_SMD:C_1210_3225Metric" (layer "B.Cu") (at 181 100 90)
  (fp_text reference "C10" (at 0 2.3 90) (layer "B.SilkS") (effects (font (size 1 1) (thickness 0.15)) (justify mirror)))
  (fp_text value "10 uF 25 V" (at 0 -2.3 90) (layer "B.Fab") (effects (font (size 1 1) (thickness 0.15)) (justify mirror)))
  (pad "1" smd roundrect (at -1.475 0 90) (size 1.15 2.7) (layers "B.Cu" "B.Paste" "B.Mask") (roundrect_rratio 0.217391) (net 1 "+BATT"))
  (pad "2" smd roundrect (at 1.475 0 90) (size 1.15 2.7) (layers "B.Cu" "B.Paste" "B.Mask") (roundrect_rratio 0.217391) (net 2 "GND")))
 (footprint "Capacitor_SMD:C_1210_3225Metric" (layer "B.Cu") (at 172 100 90)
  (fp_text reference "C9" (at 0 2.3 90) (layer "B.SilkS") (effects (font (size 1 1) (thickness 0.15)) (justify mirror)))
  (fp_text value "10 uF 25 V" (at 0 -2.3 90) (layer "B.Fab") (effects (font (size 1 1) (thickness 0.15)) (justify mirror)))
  (pad "1" smd roundrect (at -1.475 0 90) (size 1.15 2.7) (layers "B.Cu" "B.Paste" "B.Mask") (roundrect_rratio 0.217391) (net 1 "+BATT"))
  (pad "2" smd roundrect (at 1.475 0 90) (size 1.15 2.7) (layers "B.Cu" "B.Paste" "B.Mask") (roundrect_rratio 0.217391) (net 2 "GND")))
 (gr_line (start 92 90) (end 203 90) (layer "Edge.Cuts") (width 0.1))
 (gr_line (start 203 110) (end 92 110) (layer "Edge.Cuts") (width 0.1))
 (gr_line (start 92 110) (end 92 90) (layer "Edge.Cuts") (width 0.1))
 (gr_line (start 203 90) (end 203 110) (layer "Edge.Cuts") (width 0.1))
 (segment (start 95.125 103.95) (end 100 103.95) (width 0.25) (layer "F.Cu") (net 1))
 (segment (start 94 102.825) (end 95.125 103.95) (width 0.25) (layer "F.Cu") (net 1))
 (segment (start 199 101.475) (end 199 103.95) (width 2) (layer "B.Cu") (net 1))
 (segment (start 100 101.475) (end 100 103.95) (width 2) (layer "B.Cu") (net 1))
 (segment (start 145 103.95) (end 154 103.95) (width 2) (layer "B.Cu") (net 1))
 (segment (start 172 101.475) (end 172 103.95) (width 2) (layer "B.Cu") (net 1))
 (segment (start 181 103.95) (end 172 103.95) (width 2) (layer "B.Cu") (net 1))
 (segment (start 154 103.95) (end 163 103.95) (width 2) (layer "B.Cu") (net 1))
 (segment (start 109 101.475) (end 109 103.95) (width 2) (layer "B.Cu") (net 1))
 (segment (start 145 101.475) (end 145 103.95) (width 2) (layer "B.Cu") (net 1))
 (segment (start 118 101.475) (end 118 103.95) (width 2) (layer "B.Cu") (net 1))
 (segment (start 181 101.475) (end 181 103.95) (width 2) (layer "B.Cu") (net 1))
 (segment (start 190 101.475) (end 190 103.95) (width 2) (layer "B.Cu") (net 1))
 (segment (start 199 103.95) (end 190 103.95) (width 2) (layer "B.Cu") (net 1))
 (segment (start 136 101.475) (end 136 103.95) (width 2) (layer "B.Cu") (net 1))
 (segment (start 154 101.475) (end 154 103.95) (width 2) (layer "B.Cu") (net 1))
 (segment (start 118 103.95) (end 127 103.95) (width 2) (layer "B.Cu") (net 1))
 (segment (start 100 103.95) (end 109 103.95) (width 2) (layer "B.Cu") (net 1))
 (segment (start 190 103.95) (end 181 103.95) (width 2) (layer "B.Cu") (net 1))
 (segment (start 163 101.475) (end 163 103.95) (width 2) (layer "B.Cu") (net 1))
 (segment (start 136 103.95) (end 145 103.95) (width 2) (layer "B.Cu") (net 1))
 (segment (start 127 103.95) (end 136 103.95) (width 2) (layer "B.Cu") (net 1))
 (segment (start 127 101.475) (end 127 103.95) (width 2) (layer "B.Cu") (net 1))
 (segment (start 172 103.95) (end 163 103.95) (width 2) (layer "B.Cu") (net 1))
 (segment (start 109 103.95) (end 118 103.95) (width 2) (layer "B.Cu") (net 1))
 (segment (start 95.1625 96.05) (end 100 96.05) (width 0.25) (layer "F.Cu") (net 2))
 (segment (start 94 97.2125) (end 95.1625 96.05) (width 0.25) (layer "F.Cu") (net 2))
 (segment (start 136 96.05) (end 127 96.05) (width 2) (layer "B.Cu") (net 2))
 (segment (start 136 98.525) (end 136 96.05) (width 2) (layer "B.Cu") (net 2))
 (segment (start 172 96.05) (end 181 96.05) (width 2) (layer "B.Cu") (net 2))
 (segment (start 127 98.525) (end 127 96.05) (width 2) (layer "B.Cu") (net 2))
 (segment (start 190 96.05) (end 199 96.05) (width 2) (layer "B.Cu") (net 2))
 (segment (start 127 96.05) (end 118 96.05) (width 2) (layer "B.Cu") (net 2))
 (segment (start 163 98.525) (end 163 96.05) (width 2) (layer "B.Cu") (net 2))
 (segment (start 172 96.05) (end 163 96.05) (width 2) (layer "B.Cu") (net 2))
 (segment (start 145 96.05) (end 136 96.05) (width 2) (layer "B.Cu") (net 2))
 (segment (start 181 96.05) (end 190 96.05) (width 2) (layer "B.Cu") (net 2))
 (segment (start 118 98.525) (end 118 96.05) (width 2) (layer "B.Cu") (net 2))
 (segment (start 172 98.525) (end 172 96.05) (width 2) (layer "B.Cu") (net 2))
 (segment (start 163 96.05) (end 154 96.05) (width 2) (layer "B.Cu") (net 2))
 (segment (start 154 98.525) (end 154 96.05) (width 2) (layer "B.Cu") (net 2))
 (segment (start 118 96.05) (end 109 96.05) (width 2) (layer "B.Cu") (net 2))
 (segment (start 199 98.525) (end 199 96.05) (width 2) (layer "B.Cu") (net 2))
 (segment (start 154 96.05) (end 145 96.05) (width 2) (layer "B.Cu") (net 2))
 (segment (start 109 98.525) (end 109 96.05) (width 2) (layer "B.Cu") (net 2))
 (segment (start 100 98.525) (end 100 96.05) (width 2) (layer "B.Cu") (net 2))
 (segment (start 190 98.525) (end 190 96.05) (width 2) (layer "B.Cu") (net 2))
 (segment (start 109 96.05) (end 100 96.05) (width 2) (layer "B.Cu") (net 2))
 (segment (start 181 98.525) (end 181 96.05) (width 2) (layer "B.Cu") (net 2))
 (segment (start 145 98.525) (end 145 96.05) (width 2) (layer "B.Cu") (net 2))
 (segment (start 94 101.175) (end 94 98.7875) (width 0.25) (layer "F.Cu") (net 3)))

